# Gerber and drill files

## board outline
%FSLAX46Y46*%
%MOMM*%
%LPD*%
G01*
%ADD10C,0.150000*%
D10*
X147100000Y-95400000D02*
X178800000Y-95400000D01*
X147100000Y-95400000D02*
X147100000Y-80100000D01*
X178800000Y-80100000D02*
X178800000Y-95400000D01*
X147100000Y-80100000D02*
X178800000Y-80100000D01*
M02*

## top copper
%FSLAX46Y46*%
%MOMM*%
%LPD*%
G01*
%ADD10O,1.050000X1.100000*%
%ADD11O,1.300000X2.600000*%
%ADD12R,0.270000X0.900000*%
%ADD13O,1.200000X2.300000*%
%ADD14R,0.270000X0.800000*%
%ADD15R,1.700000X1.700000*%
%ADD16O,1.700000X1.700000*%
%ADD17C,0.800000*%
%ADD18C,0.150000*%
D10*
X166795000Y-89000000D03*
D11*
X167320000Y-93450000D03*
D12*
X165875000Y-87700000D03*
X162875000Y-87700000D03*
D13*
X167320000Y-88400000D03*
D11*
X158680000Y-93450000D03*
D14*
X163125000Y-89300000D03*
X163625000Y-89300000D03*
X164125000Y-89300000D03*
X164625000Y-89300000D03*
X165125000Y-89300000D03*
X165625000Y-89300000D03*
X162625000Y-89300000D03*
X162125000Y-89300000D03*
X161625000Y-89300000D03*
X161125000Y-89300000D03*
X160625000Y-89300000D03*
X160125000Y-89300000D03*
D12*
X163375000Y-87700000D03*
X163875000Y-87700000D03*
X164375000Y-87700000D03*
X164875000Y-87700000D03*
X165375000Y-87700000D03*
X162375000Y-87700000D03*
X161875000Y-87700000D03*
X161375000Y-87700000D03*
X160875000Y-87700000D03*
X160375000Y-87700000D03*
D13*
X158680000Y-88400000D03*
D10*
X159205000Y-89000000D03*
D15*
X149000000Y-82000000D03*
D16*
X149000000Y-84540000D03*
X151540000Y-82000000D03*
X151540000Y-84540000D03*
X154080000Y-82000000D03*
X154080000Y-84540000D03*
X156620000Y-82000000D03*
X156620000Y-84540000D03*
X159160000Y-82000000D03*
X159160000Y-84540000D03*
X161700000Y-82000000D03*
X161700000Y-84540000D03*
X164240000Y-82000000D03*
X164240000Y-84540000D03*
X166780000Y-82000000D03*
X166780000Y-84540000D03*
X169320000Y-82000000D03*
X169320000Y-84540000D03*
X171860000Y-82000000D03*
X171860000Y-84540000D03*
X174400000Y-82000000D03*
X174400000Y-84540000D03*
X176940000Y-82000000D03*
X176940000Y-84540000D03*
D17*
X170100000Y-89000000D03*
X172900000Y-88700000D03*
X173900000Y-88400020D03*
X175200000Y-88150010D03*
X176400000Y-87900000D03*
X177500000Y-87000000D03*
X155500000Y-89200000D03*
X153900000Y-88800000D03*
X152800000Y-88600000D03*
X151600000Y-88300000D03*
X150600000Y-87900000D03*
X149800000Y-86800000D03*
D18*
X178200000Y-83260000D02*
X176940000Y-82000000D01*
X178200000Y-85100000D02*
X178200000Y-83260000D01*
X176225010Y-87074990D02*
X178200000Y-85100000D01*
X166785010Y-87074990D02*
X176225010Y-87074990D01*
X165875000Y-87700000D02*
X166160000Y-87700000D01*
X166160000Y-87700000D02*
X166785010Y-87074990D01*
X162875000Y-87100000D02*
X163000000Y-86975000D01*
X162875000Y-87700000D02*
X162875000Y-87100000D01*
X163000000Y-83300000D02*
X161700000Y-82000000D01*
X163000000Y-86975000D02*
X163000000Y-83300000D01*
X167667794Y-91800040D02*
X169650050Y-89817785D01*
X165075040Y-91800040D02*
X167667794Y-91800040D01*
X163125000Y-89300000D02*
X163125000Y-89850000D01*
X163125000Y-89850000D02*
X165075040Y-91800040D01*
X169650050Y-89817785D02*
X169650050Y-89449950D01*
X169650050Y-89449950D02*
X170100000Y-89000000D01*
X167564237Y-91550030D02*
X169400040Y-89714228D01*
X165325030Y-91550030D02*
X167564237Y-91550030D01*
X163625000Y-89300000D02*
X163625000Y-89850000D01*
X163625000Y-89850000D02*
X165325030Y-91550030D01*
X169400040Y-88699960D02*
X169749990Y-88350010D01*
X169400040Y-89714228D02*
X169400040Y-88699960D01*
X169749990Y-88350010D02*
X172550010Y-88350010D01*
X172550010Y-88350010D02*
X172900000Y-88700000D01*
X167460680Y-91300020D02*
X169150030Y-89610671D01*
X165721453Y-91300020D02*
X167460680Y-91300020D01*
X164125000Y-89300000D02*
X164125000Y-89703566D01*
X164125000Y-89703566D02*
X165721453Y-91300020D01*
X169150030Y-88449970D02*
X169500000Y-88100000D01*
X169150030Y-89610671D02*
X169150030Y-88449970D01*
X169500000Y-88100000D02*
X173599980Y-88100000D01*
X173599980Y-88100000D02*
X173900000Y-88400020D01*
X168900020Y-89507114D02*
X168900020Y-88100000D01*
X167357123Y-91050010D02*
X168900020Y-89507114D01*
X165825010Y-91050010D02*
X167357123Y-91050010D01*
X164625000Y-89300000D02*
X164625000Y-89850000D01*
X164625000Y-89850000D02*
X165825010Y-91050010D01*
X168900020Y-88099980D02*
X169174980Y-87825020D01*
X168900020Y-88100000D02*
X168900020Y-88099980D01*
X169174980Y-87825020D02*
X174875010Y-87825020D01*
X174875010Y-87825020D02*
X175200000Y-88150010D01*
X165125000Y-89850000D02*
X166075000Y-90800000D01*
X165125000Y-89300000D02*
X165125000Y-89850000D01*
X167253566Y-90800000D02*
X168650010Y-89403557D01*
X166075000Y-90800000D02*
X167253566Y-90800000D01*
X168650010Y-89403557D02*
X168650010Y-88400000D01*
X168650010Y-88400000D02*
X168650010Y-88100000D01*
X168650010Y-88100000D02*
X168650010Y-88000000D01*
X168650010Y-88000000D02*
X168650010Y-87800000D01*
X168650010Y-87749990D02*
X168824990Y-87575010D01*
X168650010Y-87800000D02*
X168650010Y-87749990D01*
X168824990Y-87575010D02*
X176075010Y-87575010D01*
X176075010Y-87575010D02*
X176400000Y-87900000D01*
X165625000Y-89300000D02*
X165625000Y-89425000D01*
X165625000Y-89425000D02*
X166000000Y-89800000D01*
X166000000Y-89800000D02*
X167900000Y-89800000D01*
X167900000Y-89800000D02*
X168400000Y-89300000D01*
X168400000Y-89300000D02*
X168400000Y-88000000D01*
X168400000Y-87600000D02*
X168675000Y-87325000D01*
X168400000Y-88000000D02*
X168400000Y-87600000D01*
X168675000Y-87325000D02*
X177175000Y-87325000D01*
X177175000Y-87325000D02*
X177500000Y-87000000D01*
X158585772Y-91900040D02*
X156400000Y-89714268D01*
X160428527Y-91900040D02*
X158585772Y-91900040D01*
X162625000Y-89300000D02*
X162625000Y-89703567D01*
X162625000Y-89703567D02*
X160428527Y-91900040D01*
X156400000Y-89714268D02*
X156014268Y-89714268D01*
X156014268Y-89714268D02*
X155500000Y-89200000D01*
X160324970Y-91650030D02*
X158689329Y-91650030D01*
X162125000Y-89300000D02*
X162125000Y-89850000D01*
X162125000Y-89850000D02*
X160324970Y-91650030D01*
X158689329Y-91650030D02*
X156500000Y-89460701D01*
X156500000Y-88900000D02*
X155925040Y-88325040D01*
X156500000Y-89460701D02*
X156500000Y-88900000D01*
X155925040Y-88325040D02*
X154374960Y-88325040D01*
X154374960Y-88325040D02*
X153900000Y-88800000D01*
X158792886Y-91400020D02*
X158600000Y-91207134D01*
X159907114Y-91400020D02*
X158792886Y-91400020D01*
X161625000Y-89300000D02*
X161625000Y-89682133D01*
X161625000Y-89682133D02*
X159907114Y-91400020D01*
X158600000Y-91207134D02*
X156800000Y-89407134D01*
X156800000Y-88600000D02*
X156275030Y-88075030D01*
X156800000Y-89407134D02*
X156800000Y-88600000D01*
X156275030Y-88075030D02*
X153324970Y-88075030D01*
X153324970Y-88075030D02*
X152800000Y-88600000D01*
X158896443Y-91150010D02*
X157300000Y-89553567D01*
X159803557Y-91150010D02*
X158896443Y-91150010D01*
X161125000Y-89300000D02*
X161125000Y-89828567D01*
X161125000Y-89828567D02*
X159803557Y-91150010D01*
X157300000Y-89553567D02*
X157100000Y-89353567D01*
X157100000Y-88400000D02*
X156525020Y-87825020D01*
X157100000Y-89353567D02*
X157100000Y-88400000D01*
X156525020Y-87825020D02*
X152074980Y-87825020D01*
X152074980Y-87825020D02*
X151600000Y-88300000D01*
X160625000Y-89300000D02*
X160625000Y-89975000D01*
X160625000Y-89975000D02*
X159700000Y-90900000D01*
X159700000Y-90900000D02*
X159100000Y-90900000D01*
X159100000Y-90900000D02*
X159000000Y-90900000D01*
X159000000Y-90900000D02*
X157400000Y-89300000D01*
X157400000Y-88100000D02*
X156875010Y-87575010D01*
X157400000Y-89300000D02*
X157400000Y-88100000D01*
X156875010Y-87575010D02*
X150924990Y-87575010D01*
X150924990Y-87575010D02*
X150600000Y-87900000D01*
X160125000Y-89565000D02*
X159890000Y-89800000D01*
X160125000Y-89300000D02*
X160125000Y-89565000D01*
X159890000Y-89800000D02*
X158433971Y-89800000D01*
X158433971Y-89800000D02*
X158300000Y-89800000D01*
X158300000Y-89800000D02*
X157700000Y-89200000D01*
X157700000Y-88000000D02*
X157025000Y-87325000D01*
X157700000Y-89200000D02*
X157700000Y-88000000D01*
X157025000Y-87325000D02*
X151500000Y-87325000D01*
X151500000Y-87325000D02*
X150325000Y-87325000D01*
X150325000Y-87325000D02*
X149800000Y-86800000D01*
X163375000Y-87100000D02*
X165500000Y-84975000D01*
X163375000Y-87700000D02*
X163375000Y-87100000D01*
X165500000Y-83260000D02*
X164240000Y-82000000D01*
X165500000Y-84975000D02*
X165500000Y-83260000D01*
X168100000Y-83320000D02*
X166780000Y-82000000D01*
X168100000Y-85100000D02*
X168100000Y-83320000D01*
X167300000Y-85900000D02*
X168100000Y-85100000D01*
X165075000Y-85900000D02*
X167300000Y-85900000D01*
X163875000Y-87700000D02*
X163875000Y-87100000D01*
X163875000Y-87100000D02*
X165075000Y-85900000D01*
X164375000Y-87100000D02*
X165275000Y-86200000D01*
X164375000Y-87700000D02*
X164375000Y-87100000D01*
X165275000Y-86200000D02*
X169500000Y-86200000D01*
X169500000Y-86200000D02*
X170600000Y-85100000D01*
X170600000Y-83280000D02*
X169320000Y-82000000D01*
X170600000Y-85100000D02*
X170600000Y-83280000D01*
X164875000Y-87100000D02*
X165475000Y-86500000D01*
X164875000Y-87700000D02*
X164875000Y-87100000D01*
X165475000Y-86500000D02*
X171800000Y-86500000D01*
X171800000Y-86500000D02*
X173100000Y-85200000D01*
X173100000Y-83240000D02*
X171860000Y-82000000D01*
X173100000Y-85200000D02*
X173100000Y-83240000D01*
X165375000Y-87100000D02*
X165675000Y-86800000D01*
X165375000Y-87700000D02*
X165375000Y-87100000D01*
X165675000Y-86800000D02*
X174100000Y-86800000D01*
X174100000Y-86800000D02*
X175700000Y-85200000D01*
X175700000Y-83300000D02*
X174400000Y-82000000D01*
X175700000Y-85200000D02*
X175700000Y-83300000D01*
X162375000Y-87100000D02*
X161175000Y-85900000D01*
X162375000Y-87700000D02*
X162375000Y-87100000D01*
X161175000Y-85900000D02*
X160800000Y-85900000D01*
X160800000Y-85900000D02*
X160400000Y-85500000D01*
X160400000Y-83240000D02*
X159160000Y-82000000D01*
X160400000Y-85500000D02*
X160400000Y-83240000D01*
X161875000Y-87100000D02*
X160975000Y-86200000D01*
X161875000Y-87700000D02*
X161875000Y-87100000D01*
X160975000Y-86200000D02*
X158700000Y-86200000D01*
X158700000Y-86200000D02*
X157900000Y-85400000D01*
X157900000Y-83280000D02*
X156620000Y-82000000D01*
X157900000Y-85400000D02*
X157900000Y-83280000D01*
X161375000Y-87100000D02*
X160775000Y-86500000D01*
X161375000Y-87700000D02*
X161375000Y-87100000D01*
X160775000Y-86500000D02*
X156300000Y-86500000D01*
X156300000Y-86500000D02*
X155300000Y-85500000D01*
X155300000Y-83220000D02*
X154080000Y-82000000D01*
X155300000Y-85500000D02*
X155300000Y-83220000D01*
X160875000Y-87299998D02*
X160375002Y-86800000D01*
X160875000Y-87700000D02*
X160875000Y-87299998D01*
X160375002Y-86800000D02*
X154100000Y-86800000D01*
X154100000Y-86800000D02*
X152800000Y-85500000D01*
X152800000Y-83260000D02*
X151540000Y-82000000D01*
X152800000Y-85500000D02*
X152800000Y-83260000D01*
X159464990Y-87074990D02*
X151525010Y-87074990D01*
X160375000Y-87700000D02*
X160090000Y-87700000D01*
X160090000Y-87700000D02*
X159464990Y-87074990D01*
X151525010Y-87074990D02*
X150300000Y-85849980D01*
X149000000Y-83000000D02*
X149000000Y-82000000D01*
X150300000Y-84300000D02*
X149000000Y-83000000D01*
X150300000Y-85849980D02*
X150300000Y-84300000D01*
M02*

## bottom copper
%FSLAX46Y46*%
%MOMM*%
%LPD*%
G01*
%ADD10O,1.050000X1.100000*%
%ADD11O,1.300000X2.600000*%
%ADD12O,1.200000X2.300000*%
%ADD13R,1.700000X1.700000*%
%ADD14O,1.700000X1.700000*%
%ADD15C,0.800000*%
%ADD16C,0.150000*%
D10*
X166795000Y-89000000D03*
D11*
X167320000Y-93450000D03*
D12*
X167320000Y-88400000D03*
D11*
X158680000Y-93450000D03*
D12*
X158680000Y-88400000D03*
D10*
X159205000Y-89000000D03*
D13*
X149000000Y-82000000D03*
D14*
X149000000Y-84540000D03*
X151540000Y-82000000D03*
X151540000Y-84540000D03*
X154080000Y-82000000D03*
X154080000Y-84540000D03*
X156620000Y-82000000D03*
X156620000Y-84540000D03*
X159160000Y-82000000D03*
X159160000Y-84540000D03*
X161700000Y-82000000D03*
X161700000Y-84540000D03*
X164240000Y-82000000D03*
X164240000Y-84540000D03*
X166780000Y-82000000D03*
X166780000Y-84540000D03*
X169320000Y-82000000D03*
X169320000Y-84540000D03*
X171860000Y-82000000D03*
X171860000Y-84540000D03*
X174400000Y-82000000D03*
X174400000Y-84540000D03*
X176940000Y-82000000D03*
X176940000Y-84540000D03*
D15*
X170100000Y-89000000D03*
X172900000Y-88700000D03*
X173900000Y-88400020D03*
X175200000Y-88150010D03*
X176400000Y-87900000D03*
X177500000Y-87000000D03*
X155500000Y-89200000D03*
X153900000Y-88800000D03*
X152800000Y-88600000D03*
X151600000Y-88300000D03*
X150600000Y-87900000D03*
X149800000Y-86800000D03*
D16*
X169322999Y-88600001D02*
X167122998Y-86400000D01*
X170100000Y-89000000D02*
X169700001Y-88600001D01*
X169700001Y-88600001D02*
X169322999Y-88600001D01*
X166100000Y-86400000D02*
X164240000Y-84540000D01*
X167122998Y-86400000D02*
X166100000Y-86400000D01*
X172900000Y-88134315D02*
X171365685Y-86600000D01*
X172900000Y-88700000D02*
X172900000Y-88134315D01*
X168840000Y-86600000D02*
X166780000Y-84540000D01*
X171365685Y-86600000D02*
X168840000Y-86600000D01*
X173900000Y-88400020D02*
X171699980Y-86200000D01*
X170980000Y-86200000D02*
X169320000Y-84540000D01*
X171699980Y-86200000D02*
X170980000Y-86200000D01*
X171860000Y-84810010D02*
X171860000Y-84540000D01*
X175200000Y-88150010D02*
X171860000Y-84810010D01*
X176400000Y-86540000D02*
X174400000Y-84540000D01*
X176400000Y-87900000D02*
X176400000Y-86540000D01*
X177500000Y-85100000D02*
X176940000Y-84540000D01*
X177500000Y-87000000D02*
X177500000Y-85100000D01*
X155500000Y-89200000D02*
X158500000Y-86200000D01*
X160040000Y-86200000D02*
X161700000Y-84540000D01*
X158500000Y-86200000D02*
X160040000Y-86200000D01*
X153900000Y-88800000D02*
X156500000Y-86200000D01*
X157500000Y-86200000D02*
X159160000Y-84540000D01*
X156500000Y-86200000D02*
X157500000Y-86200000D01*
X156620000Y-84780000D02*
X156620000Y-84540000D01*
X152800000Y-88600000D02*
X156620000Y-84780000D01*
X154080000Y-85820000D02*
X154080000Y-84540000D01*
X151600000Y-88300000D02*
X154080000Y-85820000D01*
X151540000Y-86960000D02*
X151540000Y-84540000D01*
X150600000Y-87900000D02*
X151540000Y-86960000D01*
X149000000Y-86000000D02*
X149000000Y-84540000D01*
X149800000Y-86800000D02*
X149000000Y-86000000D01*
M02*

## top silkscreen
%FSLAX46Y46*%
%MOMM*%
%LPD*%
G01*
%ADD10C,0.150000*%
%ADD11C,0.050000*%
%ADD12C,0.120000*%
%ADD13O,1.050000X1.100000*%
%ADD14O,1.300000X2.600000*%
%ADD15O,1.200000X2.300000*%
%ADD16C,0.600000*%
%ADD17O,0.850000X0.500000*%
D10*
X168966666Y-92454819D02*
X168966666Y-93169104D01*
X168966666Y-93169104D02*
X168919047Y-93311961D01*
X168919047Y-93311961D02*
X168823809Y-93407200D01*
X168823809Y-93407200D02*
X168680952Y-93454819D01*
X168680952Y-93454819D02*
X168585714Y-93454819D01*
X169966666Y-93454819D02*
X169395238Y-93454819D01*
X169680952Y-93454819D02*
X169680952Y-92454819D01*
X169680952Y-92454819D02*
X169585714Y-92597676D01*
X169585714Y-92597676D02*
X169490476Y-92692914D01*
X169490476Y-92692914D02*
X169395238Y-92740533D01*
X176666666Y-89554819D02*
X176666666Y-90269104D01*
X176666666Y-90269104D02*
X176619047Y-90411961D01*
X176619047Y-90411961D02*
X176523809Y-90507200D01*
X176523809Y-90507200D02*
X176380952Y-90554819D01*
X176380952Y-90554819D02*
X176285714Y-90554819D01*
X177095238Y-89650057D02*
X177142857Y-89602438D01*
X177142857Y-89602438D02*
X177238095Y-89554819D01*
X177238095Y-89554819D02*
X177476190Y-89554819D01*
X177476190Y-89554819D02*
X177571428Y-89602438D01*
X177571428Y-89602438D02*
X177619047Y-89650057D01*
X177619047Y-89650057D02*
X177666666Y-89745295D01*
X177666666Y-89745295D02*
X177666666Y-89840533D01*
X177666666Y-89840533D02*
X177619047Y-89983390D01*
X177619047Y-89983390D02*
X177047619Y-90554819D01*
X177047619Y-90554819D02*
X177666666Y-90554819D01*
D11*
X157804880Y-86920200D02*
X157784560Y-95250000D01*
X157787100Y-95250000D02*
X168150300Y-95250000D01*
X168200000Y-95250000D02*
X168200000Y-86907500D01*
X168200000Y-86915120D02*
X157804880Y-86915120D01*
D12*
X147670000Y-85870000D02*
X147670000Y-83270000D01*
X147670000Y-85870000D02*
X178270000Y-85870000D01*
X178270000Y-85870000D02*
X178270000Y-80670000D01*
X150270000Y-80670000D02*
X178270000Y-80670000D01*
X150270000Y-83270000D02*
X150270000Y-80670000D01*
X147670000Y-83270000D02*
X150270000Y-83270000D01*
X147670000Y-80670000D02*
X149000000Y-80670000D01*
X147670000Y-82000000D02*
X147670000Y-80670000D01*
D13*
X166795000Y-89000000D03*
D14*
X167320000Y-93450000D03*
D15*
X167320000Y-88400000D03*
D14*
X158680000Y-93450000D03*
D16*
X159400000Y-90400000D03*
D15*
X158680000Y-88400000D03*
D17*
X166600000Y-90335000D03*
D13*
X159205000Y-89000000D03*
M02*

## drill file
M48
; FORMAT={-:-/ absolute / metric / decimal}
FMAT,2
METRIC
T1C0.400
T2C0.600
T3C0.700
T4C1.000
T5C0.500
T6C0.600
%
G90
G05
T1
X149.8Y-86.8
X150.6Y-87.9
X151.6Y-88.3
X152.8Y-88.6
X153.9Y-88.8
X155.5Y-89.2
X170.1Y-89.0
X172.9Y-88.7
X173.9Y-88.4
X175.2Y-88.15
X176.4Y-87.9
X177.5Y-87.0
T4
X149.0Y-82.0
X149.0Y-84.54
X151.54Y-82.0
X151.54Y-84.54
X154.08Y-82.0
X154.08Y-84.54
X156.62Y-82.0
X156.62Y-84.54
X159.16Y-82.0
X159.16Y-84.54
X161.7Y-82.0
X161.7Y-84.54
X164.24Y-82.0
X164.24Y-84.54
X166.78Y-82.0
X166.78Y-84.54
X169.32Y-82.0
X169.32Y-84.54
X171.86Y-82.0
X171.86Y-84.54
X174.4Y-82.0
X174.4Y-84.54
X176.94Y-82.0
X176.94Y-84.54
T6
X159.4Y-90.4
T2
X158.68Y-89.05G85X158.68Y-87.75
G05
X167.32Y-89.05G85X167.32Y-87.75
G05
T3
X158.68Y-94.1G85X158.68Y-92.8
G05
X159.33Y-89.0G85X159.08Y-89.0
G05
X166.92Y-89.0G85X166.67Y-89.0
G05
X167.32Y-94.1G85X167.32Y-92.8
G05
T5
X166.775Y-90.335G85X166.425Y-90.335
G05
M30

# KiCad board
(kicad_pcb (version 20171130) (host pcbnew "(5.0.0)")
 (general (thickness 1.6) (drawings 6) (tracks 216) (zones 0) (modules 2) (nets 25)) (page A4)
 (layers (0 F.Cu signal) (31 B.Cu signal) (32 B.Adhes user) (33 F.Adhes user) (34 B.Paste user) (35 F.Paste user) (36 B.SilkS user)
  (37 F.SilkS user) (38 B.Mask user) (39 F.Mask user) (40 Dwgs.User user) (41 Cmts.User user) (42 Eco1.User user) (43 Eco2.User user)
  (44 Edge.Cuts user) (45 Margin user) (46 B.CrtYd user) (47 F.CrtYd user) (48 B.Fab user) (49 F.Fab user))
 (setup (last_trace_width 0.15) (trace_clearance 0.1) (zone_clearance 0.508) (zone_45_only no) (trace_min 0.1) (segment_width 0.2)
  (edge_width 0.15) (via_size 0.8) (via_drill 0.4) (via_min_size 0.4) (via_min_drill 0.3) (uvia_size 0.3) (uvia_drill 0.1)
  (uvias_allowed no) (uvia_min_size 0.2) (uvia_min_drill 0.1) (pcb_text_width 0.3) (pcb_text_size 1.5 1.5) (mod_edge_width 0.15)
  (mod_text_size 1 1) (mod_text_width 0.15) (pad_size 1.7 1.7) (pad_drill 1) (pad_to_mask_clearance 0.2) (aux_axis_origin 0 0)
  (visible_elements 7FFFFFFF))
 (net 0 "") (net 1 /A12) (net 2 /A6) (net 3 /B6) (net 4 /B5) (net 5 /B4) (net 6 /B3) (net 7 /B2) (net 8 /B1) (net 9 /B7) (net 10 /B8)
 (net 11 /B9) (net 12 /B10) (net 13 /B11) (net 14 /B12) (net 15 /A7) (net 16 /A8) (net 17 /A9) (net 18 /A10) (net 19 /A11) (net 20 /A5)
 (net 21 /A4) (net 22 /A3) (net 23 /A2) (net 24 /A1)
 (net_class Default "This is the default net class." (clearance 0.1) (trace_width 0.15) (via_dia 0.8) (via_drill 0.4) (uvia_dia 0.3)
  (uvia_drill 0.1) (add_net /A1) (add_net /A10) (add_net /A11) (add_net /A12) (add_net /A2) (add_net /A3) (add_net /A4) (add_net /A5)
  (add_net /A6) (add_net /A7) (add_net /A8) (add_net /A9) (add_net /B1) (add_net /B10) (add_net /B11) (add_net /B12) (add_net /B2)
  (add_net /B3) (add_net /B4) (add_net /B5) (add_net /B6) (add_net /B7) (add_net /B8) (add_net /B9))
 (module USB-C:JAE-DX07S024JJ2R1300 (layer F.Cu) (at 159.4 90.4)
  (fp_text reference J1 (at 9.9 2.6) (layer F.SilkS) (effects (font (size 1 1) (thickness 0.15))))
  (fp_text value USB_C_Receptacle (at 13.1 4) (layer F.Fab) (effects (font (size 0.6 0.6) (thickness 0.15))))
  (fp_line (start -1.59512 -3.4798) (end -1.61544 4.85) (layer F.SilkS) (width 0.05))
  (fp_line (start -1.6129 4.85) (end 8.7503 4.85) (layer F.SilkS) (width 0.05))
  (fp_line (start 8.8 4.85) (end 8.8 -3.4925) (layer F.SilkS) (width 0.05))
  (fp_line (start 8.8 -3.48488) (end -1.59512 -3.48488) (layer F.SilkS) (width 0.05))
  (pad "" thru_hole oval (at 7.395 -1.4 180) (size 1.05 1.1) (drill oval 0.95 0.7) (layers *.Cu *.Mask F.SilkS))
  (pad "" thru_hole oval (at 7.92 3.05 90) (size 2.6 1.3) (drill oval 2 0.7) (layers *.Cu *.Mask F.SilkS))
  (pad A12 smd rect (at 6.475 -2.7) (size 0.27 0.9) (layers F.Cu F.Paste F.Mask) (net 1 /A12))
  (pad A6 smd rect (at 3.475 -2.7) (size 0.27 0.9) (layers F.Cu F.Paste F.Mask) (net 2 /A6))
  (pad "" thru_hole oval (at 7.92 -2 90) (size 2.3 1.2) (drill oval 1.9 0.6) (layers *.Cu *.Mask F.SilkS))
  (pad "" thru_hole oval (at -0.72 3.05 90) (size 2.6 1.3) (drill oval 2 0.7) (layers *.Cu *.Mask F.SilkS))
  (pad B6 smd rect (at 3.725 -1.1) (size 0.27 0.8) (layers F.Cu F.Paste F.Mask) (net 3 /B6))
  (pad B5 smd rect (at 4.225 -1.1) (size 0.27 0.8) (layers F.Cu F.Paste F.Mask) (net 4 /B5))
  (pad B4 smd rect (at 4.725 -1.1) (size 0.27 0.8) (layers F.Cu F.Paste F.Mask) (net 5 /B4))
  (pad B3 smd rect (at 5.225 -1.1) (size 0.27 0.8) (layers F.Cu F.Paste F.Mask) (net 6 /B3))
  (pad B2 smd rect (at 5.725 -1.1) (size 0.27 0.8) (layers F.Cu F.Paste F.Mask) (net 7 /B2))
  (pad B1 smd rect (at 6.225 -1.1) (size 0.27 0.8) (layers F.Cu F.Paste F.Mask) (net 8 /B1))
  (pad B7 smd rect (at 3.225 -1.1) (size 0.27 0.8) (layers F.Cu F.Paste F.Mask) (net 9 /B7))
  (pad B8 smd rect (at 2.725 -1.1) (size 0.27 0.8) (layers F.Cu F.Paste F.Mask) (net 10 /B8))
  (pad B9 smd rect (at 2.225 -1.1) (size 0.27 0.8) (layers F.Cu F.Paste F.Mask) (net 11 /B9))
  (pad B10 smd rect (at 1.725 -1.1) (size 0.27 0.8) (layers F.Cu F.Paste F.Mask) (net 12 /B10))
  (pad B11 smd rect (at 1.225 -1.1) (size 0.27 0.8) (layers F.Cu F.Paste F.Mask) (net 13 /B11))
  (pad B12 smd rect (at 0.725 -1.1) (size 0.27 0.8) (layers F.Cu F.Paste F.Mask) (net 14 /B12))
  (pad A7 smd rect (at 3.975 -2.7) (size 0.27 0.9) (layers F.Cu F.Paste F.Mask) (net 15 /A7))
  (pad A8 smd rect (at 4.475 -2.7) (size 0.27 0.9) (layers F.Cu F.Paste F.Mask) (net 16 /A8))
  (pad A9 smd rect (at 4.975 -2.7) (size 0.27 0.9) (layers F.Cu F.Paste F.Mask) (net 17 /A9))
  (pad A10 smd rect (at 5.475 -2.7) (size 0.27 0.9) (layers F.Cu F.Paste F.Mask) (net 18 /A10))
  (pad A11 smd rect (at 5.975 -2.7) (size 0.27 0.9) (layers F.Cu F.Paste F.Mask) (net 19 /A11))
  (pad A5 smd rect (at 2.975 -2.7) (size 0.27 0.9) (layers F.Cu F.Paste F.Mask) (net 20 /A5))
  (pad A4 smd rect (at 2.475 -2.7) (size 0.27 0.9) (layers F.Cu F.Paste F.Mask) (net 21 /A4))
  (pad A3 smd rect (at 1.975 -2.7) (size 0.27 0.9) (layers F.Cu F.Paste F.Mask) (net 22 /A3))
  (pad A2 smd rect (at 1.475 -2.7) (size 0.27 0.9) (layers F.Cu F.Paste F.Mask) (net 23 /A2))
  (pad A1 smd rect (at 0.975 -2.7) (size 0.27 0.9) (layers F.Cu F.Paste F.Mask) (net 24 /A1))
  (pad "" np_thru_hole circle (at 0 0 180) (size 0.6 0.6) (drill 0.6) (layers *.Cu *.Mask F.SilkS))
  (pad "" thru_hole oval (at -0.72 -2 90) (size 2.3 1.2) (drill oval 1.9 0.6) (layers *.Cu *.Mask F.SilkS))
  (pad "" np_thru_hole oval (at 7.2 -0.065 180) (size 0.85 0.5) (drill oval 0.85 0.5) (layers *.Cu *.Mask F.SilkS))
  (pad "" thru_hole oval (at -0.195 -1.4 180) (size 1.05 1.1) (drill oval 0.95 0.7) (layers *.Cu *.Mask F.SilkS)))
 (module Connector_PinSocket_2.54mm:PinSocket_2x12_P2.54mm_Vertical (layer F.Cu) (at 149 82 90)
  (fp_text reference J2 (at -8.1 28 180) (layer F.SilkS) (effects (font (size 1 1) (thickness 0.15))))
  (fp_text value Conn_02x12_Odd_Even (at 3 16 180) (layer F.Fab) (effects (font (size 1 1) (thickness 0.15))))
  (fp_line (start -3.87 -1.33) (end -1.27 -1.33) (layer F.SilkS) (width 0.12))
  (fp_line (start -3.87 -1.33) (end -3.87 29.27) (layer F.SilkS) (width 0.12))
  (fp_line (start -3.87 29.27) (end 1.33 29.27) (layer F.SilkS) (width 0.12))
  (fp_line (start 1.33 1.27) (end 1.33 29.27) (layer F.SilkS) (width 0.12))
  (fp_line (start -1.27 1.27) (end 1.33 1.27) (layer F.SilkS) (width 0.12))
  (fp_line (start -1.27 -1.33) (end -1.27 1.27) (layer F.SilkS) (width 0.12))
  (fp_line (start 1.33 -1.33) (end 1.33 0) (layer F.SilkS) (width 0.12))
  (fp_line (start 0 -1.33) (end 1.33 -1.33) (layer F.SilkS) (width 0.12))
  (pad 1 thru_hole rect (at 0 0 90) (size 1.7 1.7) (drill 1) (layers *.Cu *.Mask) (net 24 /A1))
  (pad 2 thru_hole oval (at -2.54 0 90) (size 1.7 1.7) (drill 1) (layers *.Cu *.Mask) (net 14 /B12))
  (pad 3 thru_hole oval (at 0 2.54 90) (size 1.7 1.7) (drill 1) (layers *.Cu *.Mask) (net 23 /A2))
  (pad 4 thru_hole oval (at -2.54 2.54 90) (size 1.7 1.7) (drill 1) (layers *.Cu *.Mask) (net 13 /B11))
  (pad 5 thru_hole oval (at 0 5.08 90) (size 1.7 1.7) (drill 1) (layers *.Cu *.Mask) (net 22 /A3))
  (pad 6 thru_hole oval (at -2.54 5.08 90) (size 1.7 1.7) (drill 1) (layers *.Cu *.Mask) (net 12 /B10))
  (pad 7 thru_hole oval (at 0 7.62 90) (size 1.7 1.7) (drill 1) (layers *.Cu *.Mask) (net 21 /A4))
  (pad 8 thru_hole oval (at -2.54 7.62 90) (size 1.7 1.7) (drill 1) (layers *.Cu *.Mask) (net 11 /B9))
  (pad 9 thru_hole oval (at 0 10.16 90) (size 1.7 1.7) (drill 1) (layers *.Cu *.Mask) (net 20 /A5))
  (pad 10 thru_hole oval (at -2.54 10.16 90) (size 1.7 1.7) (drill 1) (layers *.Cu *.Mask) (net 10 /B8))
  (pad 11 thru_hole oval (at 0 12.7 90) (size 1.7 1.7) (drill 1) (layers *.Cu *.Mask) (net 2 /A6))
  (pad 12 thru_hole oval (at -2.54 12.7 90) (size 1.7 1.7) (drill 1) (layers *.Cu *.Mask) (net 9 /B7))
  (pad 13 thru_hole oval (at 0 15.24 90) (size 1.7 1.7) (drill 1) (layers *.Cu *.Mask) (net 15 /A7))
  (pad 14 thru_hole oval (at -2.54 15.24 90) (size 1.7 1.7) (drill 1) (layers *.Cu *.Mask) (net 3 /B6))
  (pad 15 thru_hole oval (at 0 17.78 90) (size 1.7 1.7) (drill 1) (layers *.Cu *.Mask) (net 16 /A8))
  (pad 16 thru_hole oval (at -2.54 17.78 90) (size 1.7 1.7) (drill 1) (layers *.Cu *.Mask) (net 4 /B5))
  (pad 17 thru_hole oval (at 0 20.32 90) (size 1.7 1.7) (drill 1) (layers *.Cu *.Mask) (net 17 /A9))
  (pad 18 thru_hole oval (at -2.54 20.32 90) (size 1.7 1.7) (drill 1) (layers *.Cu *.Mask) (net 5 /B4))
  (pad 19 thru_hole oval (at 0 22.86 90) (size 1.7 1.7) (drill 1) (layers *.Cu *.Mask) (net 18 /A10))
  (pad 20 thru_hole oval (at -2.54 22.86 90) (size 1.7 1.7) (drill 1) (layers *.Cu *.Mask) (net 6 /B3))
  (pad 21 thru_hole oval (at 0 25.4 90) (size 1.7 1.7) (drill 1) (layers *.Cu *.Mask) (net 19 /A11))
  (pad 22 thru_hole oval (at -2.54 25.4 90) (size 1.7 1.7) (drill 1) (layers *.Cu *.Mask) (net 7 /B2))
  (pad 23 thru_hole oval (at 0 27.94 90) (size 1.7 1.7) (drill 1) (layers *.Cu *.Mask) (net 1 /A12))
  (pad 24 thru_hole oval (at -2.54 27.94 90) (size 1.7 1.7) (drill 1) (layers *.Cu *.Mask) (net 8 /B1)))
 (gr_line (start 147.1 95.4) (end 178.8 95.4) (layer Edge.Cuts) (width 0.15))
 (gr_line (start 147.1 95.4) (end 147.1 80.1) (layer Edge.Cuts) (width 0.15))
 (gr_line (start 178.8 80.1) (end 178.8 95.4) (layer Edge.Cuts) (width 0.15))
 (gr_line (start 147.1 80.1) (end 178.8 80.1) (layer Edge.Cuts) (width 0.15))
 (segment (start 178.2 83.26) (end 176.94 82) (width 0.15) (layer F.Cu) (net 1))
 (segment (start 178.2 85.1) (end 178.2 83.26) (width 0.15) (layer F.Cu) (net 1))
 (segment (start 176.22501 87.07499) (end 178.2 85.1) (width 0.15) (layer F.Cu) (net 1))
 (segment (start 166.78501 87.07499) (end 176.22501 87.07499) (width 0.15) (layer F.Cu) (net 1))
 (segment (start 165.875 87.7) (end 166.16 87.7) (width 0.15) (layer F.Cu) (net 1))
 (segment (start 166.16 87.7) (end 166.78501 87.07499) (width 0.15) (layer F.Cu) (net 1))
 (segment (start 162.875 87.1) (end 163 86.975) (width 0.15) (layer F.Cu) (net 2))
 (segment (start 162.875 87.7) (end 162.875 87.1) (width 0.15) (layer F.Cu) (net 2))
 (segment (start 163 83.3) (end 161.7 82) (width 0.15) (layer F.Cu) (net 2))
 (segment (start 163 86.975) (end 163 83.3) (width 0.15) (layer F.Cu) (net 2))
 (segment (start 167.667794 91.80004) (end 169.65005 89.817785) (width 0.15) (layer F.Cu) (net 3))
 (segment (start 165.07504 91.80004) (end 167.667794 91.80004) (width 0.15) (layer F.Cu) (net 3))
 (segment (start 163.125 89.3) (end 163.125 89.85) (width 0.15) (layer F.Cu) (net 3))
 (segment (start 163.125 89.85) (end 165.07504 91.80004) (width 0.15) (layer F.Cu) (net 3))
 (via (at 170.1 89) (size 0.8) (drill 0.4) (layers F.Cu B.Cu) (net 3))
 (segment (start 169.65005 89.817785) (end 169.65005 89.44995) (width 0.15) (layer F.Cu) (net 3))
 (segment (start 169.65005 89.44995) (end 170.1 89) (width 0.15) (layer F.Cu) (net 3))
 (segment (start 169.322999 88.600001) (end 167.122998 86.4) (width 0.15) (layer B.Cu) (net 3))
 (segment (start 170.1 89) (end 169.700001 88.600001) (width 0.15) (layer B.Cu) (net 3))
 (segment (start 169.700001 88.600001) (end 169.322999 88.600001) (width 0.15) (layer B.Cu) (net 3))
 (segment (start 166.1 86.4) (end 164.24 84.54) (width 0.15) (layer B.Cu) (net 3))
 (segment (start 167.122998 86.4) (end 166.1 86.4) (width 0.15) (layer B.Cu) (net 3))
 (segment (start 167.564237 91.55003) (end 169.40004 89.714228) (width 0.15) (layer F.Cu) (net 4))
 (segment (start 165.32503 91.55003) (end 167.564237 91.55003) (width 0.15) (layer F.Cu) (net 4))
 (segment (start 163.625 89.3) (end 163.625 89.85) (width 0.15) (layer F.Cu) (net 4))
 (segment (start 163.625 89.85) (end 165.32503 91.55003) (width 0.15) (layer F.Cu) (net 4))
 (segment (start 169.40004 88.69996) (end 169.74999 88.35001) (width 0.15) (layer F.Cu) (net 4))
 (segment (start 169.40004 89.714228) (end 169.40004 88.69996) (width 0.15) (layer F.Cu) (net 4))
 (via (at 172.9 88.7) (size 0.8) (drill 0.4) (layers F.Cu B.Cu) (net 4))
 (segment (start 169.74999 88.35001) (end 172.55001 88.35001) (width 0.15) (layer F.Cu) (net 4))
 (segment (start 172.55001 88.35001) (end 172.9 88.7) (width 0.15) (layer F.Cu) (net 4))
 (segment (start 172.9 88.134315) (end 171.365685 86.6) (width 0.15) (layer B.Cu) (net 4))
 (segment (start 172.9 88.7) (end 172.9 88.134315) (width 0.15) (layer B.Cu) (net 4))
 (segment (start 168.84 86.6) (end 166.78 84.54) (width 0.15) (layer B.Cu) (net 4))
 (segment (start 171.365685 86.6) (end 168.84 86.6) (width 0.15) (layer B.Cu) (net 4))
 (segment (start 167.46068 91.30002) (end 169.15003 89.610671) (width 0.15) (layer F.Cu) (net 5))
 (segment (start 165.721453 91.30002) (end 167.46068 91.30002) (width 0.15) (layer F.Cu) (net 5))
 (segment (start 164.125 89.3) (end 164.125 89.703566) (width 0.15) (layer F.Cu) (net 5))
 (segment (start 164.125 89.703566) (end 165.721453 91.30002) (width 0.15) (layer F.Cu) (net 5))
 (segment (start 169.15003 88.44997) (end 169.5 88.1) (width 0.15) (layer F.Cu) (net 5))
 (segment (start 169.15003 89.610671) (end 169.15003 88.44997) (width 0.15) (layer F.Cu) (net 5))
 (via (at 173.9 88.40002) (size 0.8) (drill 0.4) (layers F.Cu B.Cu) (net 5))
 (segment (start 169.5 88.1) (end 173.59998 88.1) (width 0.15) (layer F.Cu) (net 5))
 (segment (start 173.59998 88.1) (end 173.9 88.40002) (width 0.15) (layer F.Cu) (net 5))
 (segment (start 173.9 88.40002) (end 171.69998 86.2) (width 0.15) (layer B.Cu) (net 5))
 (segment (start 170.98 86.2) (end 169.32 84.54) (width 0.15) (layer B.Cu) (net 5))
 (segment (start 171.69998 86.2) (end 170.98 86.2) (width 0.15) (layer B.Cu) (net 5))
 (segment (start 168.90002 89.507114) (end 168.90002 88.1) (width 0.15) (layer F.Cu) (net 6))
 (segment (start 167.357123 91.05001) (end 168.90002 89.507114) (width 0.15) (layer F.Cu) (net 6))
 (segment (start 165.82501 91.05001) (end 167.357123 91.05001) (width 0.15) (layer F.Cu) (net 6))
 (segment (start 164.625 89.3) (end 164.625 89.85) (width 0.15) (layer F.Cu) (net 6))
 (segment (start 164.625 89.85) (end 165.82501 91.05001) (width 0.15) (layer F.Cu) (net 6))
 (segment (start 168.90002 88.09998) (end 169.17498 87.82502) (width 0.15) (layer F.Cu) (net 6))
 (segment (start 168.90002 88.1) (end 168.90002 88.09998) (width 0.15) (layer F.Cu) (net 6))
 (via (at 175.2 88.15001) (size 0.8) (drill 0.4) (layers F.Cu B.Cu) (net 6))
 (segment (start 169.17498 87.82502) (end 174.87501 87.82502) (width 0.15) (layer F.Cu) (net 6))
 (segment (start 174.87501 87.82502) (end 175.2 88.15001) (width 0.15) (layer F.Cu) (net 6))
 (segment (start 171.86 84.81001) (end 171.86 84.54) (width 0.15) (layer B.Cu) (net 6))
 (segment (start 175.2 88.15001) (end 171.86 84.81001) (width 0.15) (layer B.Cu) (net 6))
 (segment (start 165.125 89.85) (end 166.075 90.8) (width 0.15) (layer F.Cu) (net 7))
 (segment (start 165.125 89.3) (end 165.125 89.85) (width 0.15) (layer F.Cu) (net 7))
 (segment (start 167.253566 90.8) (end 168.65001 89.403557) (width 0.15) (layer F.Cu) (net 7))
 (segment (start 166.075 90.8) (end 167.253566 90.8) (width 0.15) (layer F.Cu) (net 7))
 (segment (start 168.65001 89.403557) (end 168.65001 88.4) (width 0.15) (layer F.Cu) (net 7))
 (segment (start 168.65001 88.4) (end 168.65001 88.1) (width 0.15) (layer F.Cu) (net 7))
 (segment (start 168.65001 88.1) (end 168.65001 88) (width 0.15) (layer F.Cu) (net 7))
 (segment (start 168.65001 88) (end 168.65001 87.8) (width 0.15) (layer F.Cu) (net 7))
 (segment (start 168.65001 87.74999) (end 168.82499 87.57501) (width 0.15) (layer F.Cu) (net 7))
 (segment (start 168.65001 87.8) (end 168.65001 87.74999) (width 0.15) (layer F.Cu) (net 7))
 (via (at 176.4 87.9) (size 0.8) (drill 0.4) (layers F.Cu B.Cu) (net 7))
 (segment (start 168.82499 87.57501) (end 176.07501 87.57501) (width 0.15) (layer F.Cu) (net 7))
 (segment (start 176.07501 87.57501) (end 176.4 87.9) (width 0.15) (layer F.Cu) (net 7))
 (segment (start 176.4 86.54) (end 174.4 84.54) (width 0.15) (layer B.Cu) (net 7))
 (segment (start 176.4 87.9) (end 176.4 86.54) (width 0.15) (layer B.Cu) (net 7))
 (segment (start 165.625 89.3) (end 165.625 89.425) (width 0.15) (layer F.Cu) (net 8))
 (segment (start 165.625 89.425) (end 166 89.8) (width 0.15) (layer F.Cu) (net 8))
 (segment (start 166 89.8) (end 167.9 89.8) (width 0.15) (layer F.Cu) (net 8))
 (segment (start 167.9 89.8) (end 168.4 89.3) (width 0.15) (layer F.Cu) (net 8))
 (segment (start 168.4 89.3) (end 168.4 88) (width 0.15) (layer F.Cu) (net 8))
 (segment (start 168.4 87.6) (end 168.675 87.325) (width 0.15) (layer F.Cu) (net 8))
 (segment (start 168.4 88) (end 168.4 87.6) (width 0.15) (layer F.Cu) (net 8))
 (via (at 177.5 87) (size 0.8) (drill 0.4) (layers F.Cu B.Cu) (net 8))
 (segment (start 168.675 87.325) (end 177.175 87.325) (width 0.15) (layer F.Cu) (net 8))
 (segment (start 177.175 87.325) (end 177.5 87) (width 0.15) (layer F.Cu) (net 8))
 (segment (start 177.5 85.1) (end 176.94 84.54) (width 0.15) (layer B.Cu) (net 8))
 (segment (start 177.5 87) (end 177.5 85.1) (width 0.15) (layer B.Cu) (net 8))
 (segment (start 158.585772 91.90004) (end 156.4 89.714268) (width 0.15) (layer F.Cu) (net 9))
 (segment (start 160.428527 91.90004) (end 158.585772 91.90004) (width 0.15) (layer F.Cu) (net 9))
 (segment (start 162.625 89.3) (end 162.625 89.703567) (width 0.15) (layer F.Cu) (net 9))
 (segment (start 162.625 89.703567) (end 160.428527 91.90004) (width 0.15) (layer F.Cu) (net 9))
 (via (at 155.5 89.2) (size 0.8) (drill 0.4) (layers F.Cu B.Cu) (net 9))
 (segment (start 156.4 89.714268) (end 156.014268 89.714268) (width 0.15) (layer F.Cu) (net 9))
 (segment (start 156.014268 89.714268) (end 155.5 89.2) (width 0.15) (layer F.Cu) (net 9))
 (segment (start 155.5 89.2) (end 158.5 86.2) (width 0.15) (layer B.Cu) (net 9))
 (segment (start 160.04 86.2) (end 161.7 84.54) (width 0.15) (layer B.Cu) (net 9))
 (segment (start 158.5 86.2) (end 160.04 86.2) (width 0.15) (layer B.Cu) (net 9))
 (segment (start 160.32497 91.65003) (end 158.689329 91.65003) (width 0.15) (layer F.Cu) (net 10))
 (segment (start 162.125 89.3) (end 162.125 89.85) (width 0.15) (layer F.Cu) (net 10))
 (segment (start 162.125 89.85) (end 160.32497 91.65003) (width 0.15) (layer F.Cu) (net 10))
 (segment (start 158.689329 91.65003) (end 156.5 89.460701) (width 0.15) (layer F.Cu) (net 10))
 (segment (start 156.5 88.9) (end 155.92504 88.32504) (width 0.15) (layer F.Cu) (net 10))
 (segment (start 156.5 89.460701) (end 156.5 88.9) (width 0.15) (layer F.Cu) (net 10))
 (via (at 153.9 88.8) (size 0.8) (drill 0.4) (layers F.Cu B.Cu) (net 10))
 (segment (start 155.92504 88.32504) (end 154.37496 88.32504) (width 0.15) (layer F.Cu) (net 10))
 (segment (start 154.37496 88.32504) (end 153.9 88.8) (width 0.15) (layer F.Cu) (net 10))
 (segment (start 153.9 88.8) (end 156.5 86.2) (width 0.15) (layer B.Cu) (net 10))
 (segment (start 157.5 86.2) (end 159.16 84.54) (width 0.15) (layer B.Cu) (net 10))
 (segment (start 156.5 86.2) (end 157.5 86.2) (width 0.15) (layer B.Cu) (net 10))
 (segment (start 158.792886 91.40002) (end 158.6 91.207134) (width 0.15) (layer F.Cu) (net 11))
 (segment (start 159.907114 91.40002) (end 158.792886 91.40002) (width 0.15) (layer F.Cu) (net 11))
 (segment (start 161.625 89.3) (end 161.625 89.682133) (width 0.15) (layer F.Cu) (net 11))
 (segment (start 161.625 89.682133) (end 159.907114 91.40002) (width 0.15) (layer F.Cu) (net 11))
 (segment (start 158.6 91.207134) (end 156.8 89.407134) (width 0.15) (layer F.Cu) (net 11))
 (segment (start 156.8 88.6) (end 156.27503 88.07503) (width 0.15) (layer F.Cu) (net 11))
 (segment (start 156.8 89.407134) (end 156.8 88.6) (width 0.15) (layer F.Cu) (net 11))
 (via (at 152.8 88.6) (size 0.8) (drill 0.4) (layers F.Cu B.Cu) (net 11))
 (segment (start 156.27503 88.07503) (end 153.32497 88.07503) (width 0.15) (layer F.Cu) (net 11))
 (segment (start 153.32497 88.07503) (end 152.8 88.6) (width 0.15) (layer F.Cu) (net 11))
 (segment (start 156.62 84.78) (end 156.62 84.54) (width 0.15) (layer B.Cu) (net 11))
 (segment (start 152.8 88.6) (end 156.62 84.78) (width 0.15) (layer B.Cu) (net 11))
 (segment (start 158.896443 91.15001) (end 157.3 89.553567) (width 0.15) (layer F.Cu) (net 12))
 (segment (start 159.803557 91.15001) (end 158.896443 91.15001) (width 0.15) (layer F.Cu) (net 12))
 (segment (start 161.125 89.3) (end 161.125 89.828567) (width 0.15) (layer F.Cu) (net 12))
 (segment (start 161.125 89.828567) (end 159.803557 91.15001) (width 0.15) (layer F.Cu) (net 12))
 (segment (start 157.3 89.553567) (end 157.1 89.353567) (width 0.15) (layer F.Cu) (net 12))
 (segment (start 157.1 88.4) (end 156.52502 87.82502) (width 0.15) (layer F.Cu) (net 12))
 (segment (start 157.1 89.353567) (end 157.1 88.4) (width 0.15) (layer F.Cu) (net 12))
 (via (at 151.6 88.3) (size 0.8) (drill 0.4) (layers F.Cu B.Cu) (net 12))
 (segment (start 156.52502 87.82502) (end 152.07498 87.82502) (width 0.15) (layer F.Cu) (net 12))
 (segment (start 152.07498 87.82502) (end 151.6 88.3) (width 0.15) (layer F.Cu) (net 12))
 (segment (start 154.08 85.82) (end 154.08 84.54) (width 0.15) (layer B.Cu) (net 12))
 (segment (start 151.6 88.3) (end 154.08 85.82) (width 0.15) (layer B.Cu) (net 12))
 (segment (start 160.625 89.3) (end 160.625 89.975) (width 0.15) (layer F.Cu) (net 13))
 (segment (start 160.625 89.975) (end 159.7 90.9) (width 0.15) (layer F.Cu) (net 13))
 (segment (start 159.7 90.9) (end 159.1 90.9) (width 0.15) (layer F.Cu) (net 13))
 (segment (start 159.1 90.9) (end 159 90.9) (width 0.15) (layer F.Cu) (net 13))
 (segment (start 159 90.9) (end 157.4 89.3) (width 0.15) (layer F.Cu) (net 13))
 (segment (start 157.4 88.1) (end 156.87501 87.57501) (width 0.15) (layer F.Cu) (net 13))
 (segment (start 157.4 89.3) (end 157.4 88.1) (width 0.15) (layer F.Cu) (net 13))
 (via (at 150.6 87.9) (size 0.8) (drill 0.4) (layers F.Cu B.Cu) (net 13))
 (segment (start 156.87501 87.57501) (end 150.92499 87.57501) (width 0.15) (layer F.Cu) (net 13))
 (segment (start 150.92499 87.57501) (end 150.6 87.9) (width 0.15) (layer F.Cu) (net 13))
 (segment (start 151.54 86.96) (end 151.54 84.54) (width 0.15) (layer B.Cu) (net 13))
 (segment (start 150.6 87.9) (end 151.54 86.96) (width 0.15) (layer B.Cu) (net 13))
 (segment (start 160.125 89.565) (end 159.89 89.8) (width 0.15) (layer F.Cu) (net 14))
 (segment (start 160.125 89.3) (end 160.125 89.565) (width 0.15) (layer F.Cu) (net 14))
 (segment (start 159.89 89.8) (end 158.433971 89.8) (width 0.15) (layer F.Cu) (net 14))
 (segment (start 158.433971 89.8) (end 158.3 89.8) (width 0.15) (layer F.Cu) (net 14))
 (segment (start 158.3 89.8) (end 157.7 89.2) (width 0.15) (layer F.Cu) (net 14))
 (segment (start 157.7 88) (end 157.025 87.325) (width 0.15) (layer F.Cu) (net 14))
 (segment (start 157.7 89.2) (end 157.7 88) (width 0.15) (layer F.Cu) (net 14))
 (segment (start 157.025 87.325) (end 151.5 87.325) (width 0.15) (layer F.Cu) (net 14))
 (via (at 149.8 86.8) (size 0.8) (drill 0.4) (layers F.Cu B.Cu) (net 14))
 (segment (start 151.5 87.325) (end 150.325 87.325) (width 0.15) (layer F.Cu) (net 14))
 (segment (start 150.325 87.325) (end 149.8 86.8) (width 0.15) (layer F.Cu) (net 14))
 (segment (start 149 86) (end 149 84.54) (width 0.15) (layer B.Cu) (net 14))
 (segment (start 149.8 86.8) (end 149 86) (width 0.15) (layer B.Cu) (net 14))
 (segment (start 163.375 87.1) (end 165.5 84.975) (width 0.15) (layer F.Cu) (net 15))
 (segment (start 163.375 87.7) (end 163.375 87.1) (width 0.15) (layer F.Cu) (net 15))
 (segment (start 165.5 83.26) (end 164.24 82) (width 0.15) (layer F.Cu) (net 15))
 (segment (start 165.5 84.975) (end 165.5 83.26) (width 0.15) (layer F.Cu) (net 15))
 (segment (start 168.1 83.32) (end 166.78 82) (width 0.15) (layer F.Cu) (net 16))
 (segment (start 168.1 85.1) (end 168.1 83.32) (width 0.15) (layer F.Cu) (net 16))
 (segment (start 167.3 85.9) (end 168.1 85.1) (width 0.15) (layer F.Cu) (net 16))
 (segment (start 165.075 85.9) (end 167.3 85.9) (width 0.15) (layer F.Cu) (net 16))
 (segment (start 163.875 87.7) (end 163.875 87.1) (width 0.15) (layer F.Cu) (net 16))
 (segment (start 163.875 87.1) (end 165.075 85.9) (width 0.15) (layer F.Cu) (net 16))
 (segment (start 164.375 87.1) (end 165.275 86.2) (width 0.15) (layer F.Cu) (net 17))
 (segment (start 164.375 87.7) (end 164.375 87.1) (width 0.15) (layer F.Cu) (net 17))
 (segment (start 165.275 86.2) (end 169.5 86.2) (width 0.15) (layer F.Cu) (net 17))
 (segment (start 169.5 86.2) (end 170.6 85.1) (width 0.15) (layer F.Cu) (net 17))
 (segment (start 170.6 83.28) (end 169.32 82) (width 0.15) (layer F.Cu) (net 17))
 (segment (start 170.6 85.1) (end 170.6 83.28) (width 0.15) (layer F.Cu) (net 17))
 (segment (start 164.875 87.1) (end 165.475 86.5) (width 0.15) (layer F.Cu) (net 18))
 (segment (start 164.875 87.7) (end 164.875 87.1) (width 0.15) (layer F.Cu) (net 18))
 (segment (start 165.475 86.5) (end 171.8 86.5) (width 0.15) (layer F.Cu) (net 18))
 (segment (start 171.8 86.5) (end 173.1 85.2) (width 0.15) (layer F.Cu) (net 18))
 (segment (start 173.1 83.24) (end 171.86 82) (width 0.15) (layer F.Cu) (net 18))
 (segment (start 173.1 85.2) (end 173.1 83.24) (width 0.15) (layer F.Cu) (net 18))
 (segment (start 165.375 87.1) (end 165.675 86.8) (width 0.15) (layer F.Cu) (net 19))
 (segment (start 165.375 87.7) (end 165.375 87.1) (width 0.15) (layer F.Cu) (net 19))
 (segment (start 165.675 86.8) (end 174.1 86.8) (width 0.15) (layer F.Cu) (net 19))
 (segment (start 174.1 86.8) (end 175.7 85.2) (width 0.15) (layer F.Cu) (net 19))
 (segment (start 175.7 83.3) (end 174.4 82) (width 0.15) (layer F.Cu) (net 19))
 (segment (start 175.7 85.2) (end 175.7 83.3) (width 0.15) (layer F.Cu) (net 19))
 (segment (start 162.375 87.1) (end 161.175 85.9) (width 0.15) (layer F.Cu) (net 20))
 (segment (start 162.375 87.7) (end 162.375 87.1) (width 0.15) (layer F.Cu) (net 20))
 (segment (start 161.175 85.9) (end 160.8 85.9) (width 0.15) (layer F.Cu) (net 20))
 (segment (start 160.8 85.9) (end 160.4 85.5) (width 0.15) (layer F.Cu) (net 20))
 (segment (start 160.4 83.24) (end 159.16 82) (width 0.15) (layer F.Cu) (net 20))
 (segment (start 160.4 85.5) (end 160.4 83.24) (width 0.15) (layer F.Cu) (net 20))
 (segment (start 161.875 87.1) (end 160.975 86.2) (width 0.15) (layer F.Cu) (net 21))
 (segment (start 161.875 87.7) (end 161.875 87.1) (width 0.15) (layer F.Cu) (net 21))
 (segment (start 160.975 86.2) (end 158.7 86.2) (width 0.15) (layer F.Cu) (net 21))
 (segment (start 158.7 86.2) (end 157.9 85.4) (width 0.15) (layer F.Cu) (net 21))
 (segment (start 157.9 83.28) (end 156.62 82) (width 0.15) (layer F.Cu) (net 21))
 (segment (start 157.9 85.4) (end 157.9 83.28) (width 0.15) (layer F.Cu) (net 21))
 (segment (start 161.375 87.1) (end 160.775 86.5) (width 0.15) (layer F.Cu) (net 22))
 (segment (start 161.375 87.7) (end 161.375 87.1) (width 0.15) (layer F.Cu) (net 22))
 (segment (start 160.775 86.5) (end 156.3 86.5) (width 0.15) (layer F.Cu) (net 22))
 (segment (start 156.3 86.5) (end 155.3 85.5) (width 0.15) (layer F.Cu) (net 22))
 (segment (start 155.3 83.22) (end 154.08 82) (width 0.15) (layer F.Cu) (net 22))
 (segment (start 155.3 85.5) (end 155.3 83.22) (width 0.15) (layer F.Cu) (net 22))
 (segment (start 160.875 87.299998) (end 160.375002 86.8) (width 0.15) (layer F.Cu) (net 23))
 (segment (start 160.875 87.7) (end 160.875 87.299998) (width 0.15) (layer F.Cu) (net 23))
 (segment (start 160.375002 86.8) (end 154.1 86.8) (width 0.15) (layer F.Cu) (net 23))
 (segment (start 154.1 86.8) (end 152.8 85.5) (width 0.15) (layer F.Cu) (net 23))
 (segment (start 152.8 83.26) (end 151.54 82) (width 0.15) (layer F.Cu) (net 23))
 (segment (start 152.8 85.5) (end 152.8 83.26) (width 0.15) (layer F.Cu) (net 23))
 (segment (start 159.46499 87.07499) (end 151.52501 87.07499) (width 0.15) (layer F.Cu) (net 24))
 (segment (start 160.375 87.7) (end 160.09 87.7) (width 0.15) (layer F.Cu) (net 24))
 (segment (start 160.09 87.7) (end 159.46499 87.07499) (width 0.15) (layer F.Cu) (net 24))
 (segment (start 151.52501 87.07499) (end 150.3 85.84998) (width 0.15) (layer F.Cu) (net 24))
 (segment (start 149 83) (end 149 82) (width 0.15) (layer F.Cu) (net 24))
 (segment (start 150.3 84.3) (end 149 83) (width 0.15) (layer F.Cu) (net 24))
 (segment (start 150.3 85.84998) (end 150.3 84.3) (width 0.15) (layer F.Cu) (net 24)))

